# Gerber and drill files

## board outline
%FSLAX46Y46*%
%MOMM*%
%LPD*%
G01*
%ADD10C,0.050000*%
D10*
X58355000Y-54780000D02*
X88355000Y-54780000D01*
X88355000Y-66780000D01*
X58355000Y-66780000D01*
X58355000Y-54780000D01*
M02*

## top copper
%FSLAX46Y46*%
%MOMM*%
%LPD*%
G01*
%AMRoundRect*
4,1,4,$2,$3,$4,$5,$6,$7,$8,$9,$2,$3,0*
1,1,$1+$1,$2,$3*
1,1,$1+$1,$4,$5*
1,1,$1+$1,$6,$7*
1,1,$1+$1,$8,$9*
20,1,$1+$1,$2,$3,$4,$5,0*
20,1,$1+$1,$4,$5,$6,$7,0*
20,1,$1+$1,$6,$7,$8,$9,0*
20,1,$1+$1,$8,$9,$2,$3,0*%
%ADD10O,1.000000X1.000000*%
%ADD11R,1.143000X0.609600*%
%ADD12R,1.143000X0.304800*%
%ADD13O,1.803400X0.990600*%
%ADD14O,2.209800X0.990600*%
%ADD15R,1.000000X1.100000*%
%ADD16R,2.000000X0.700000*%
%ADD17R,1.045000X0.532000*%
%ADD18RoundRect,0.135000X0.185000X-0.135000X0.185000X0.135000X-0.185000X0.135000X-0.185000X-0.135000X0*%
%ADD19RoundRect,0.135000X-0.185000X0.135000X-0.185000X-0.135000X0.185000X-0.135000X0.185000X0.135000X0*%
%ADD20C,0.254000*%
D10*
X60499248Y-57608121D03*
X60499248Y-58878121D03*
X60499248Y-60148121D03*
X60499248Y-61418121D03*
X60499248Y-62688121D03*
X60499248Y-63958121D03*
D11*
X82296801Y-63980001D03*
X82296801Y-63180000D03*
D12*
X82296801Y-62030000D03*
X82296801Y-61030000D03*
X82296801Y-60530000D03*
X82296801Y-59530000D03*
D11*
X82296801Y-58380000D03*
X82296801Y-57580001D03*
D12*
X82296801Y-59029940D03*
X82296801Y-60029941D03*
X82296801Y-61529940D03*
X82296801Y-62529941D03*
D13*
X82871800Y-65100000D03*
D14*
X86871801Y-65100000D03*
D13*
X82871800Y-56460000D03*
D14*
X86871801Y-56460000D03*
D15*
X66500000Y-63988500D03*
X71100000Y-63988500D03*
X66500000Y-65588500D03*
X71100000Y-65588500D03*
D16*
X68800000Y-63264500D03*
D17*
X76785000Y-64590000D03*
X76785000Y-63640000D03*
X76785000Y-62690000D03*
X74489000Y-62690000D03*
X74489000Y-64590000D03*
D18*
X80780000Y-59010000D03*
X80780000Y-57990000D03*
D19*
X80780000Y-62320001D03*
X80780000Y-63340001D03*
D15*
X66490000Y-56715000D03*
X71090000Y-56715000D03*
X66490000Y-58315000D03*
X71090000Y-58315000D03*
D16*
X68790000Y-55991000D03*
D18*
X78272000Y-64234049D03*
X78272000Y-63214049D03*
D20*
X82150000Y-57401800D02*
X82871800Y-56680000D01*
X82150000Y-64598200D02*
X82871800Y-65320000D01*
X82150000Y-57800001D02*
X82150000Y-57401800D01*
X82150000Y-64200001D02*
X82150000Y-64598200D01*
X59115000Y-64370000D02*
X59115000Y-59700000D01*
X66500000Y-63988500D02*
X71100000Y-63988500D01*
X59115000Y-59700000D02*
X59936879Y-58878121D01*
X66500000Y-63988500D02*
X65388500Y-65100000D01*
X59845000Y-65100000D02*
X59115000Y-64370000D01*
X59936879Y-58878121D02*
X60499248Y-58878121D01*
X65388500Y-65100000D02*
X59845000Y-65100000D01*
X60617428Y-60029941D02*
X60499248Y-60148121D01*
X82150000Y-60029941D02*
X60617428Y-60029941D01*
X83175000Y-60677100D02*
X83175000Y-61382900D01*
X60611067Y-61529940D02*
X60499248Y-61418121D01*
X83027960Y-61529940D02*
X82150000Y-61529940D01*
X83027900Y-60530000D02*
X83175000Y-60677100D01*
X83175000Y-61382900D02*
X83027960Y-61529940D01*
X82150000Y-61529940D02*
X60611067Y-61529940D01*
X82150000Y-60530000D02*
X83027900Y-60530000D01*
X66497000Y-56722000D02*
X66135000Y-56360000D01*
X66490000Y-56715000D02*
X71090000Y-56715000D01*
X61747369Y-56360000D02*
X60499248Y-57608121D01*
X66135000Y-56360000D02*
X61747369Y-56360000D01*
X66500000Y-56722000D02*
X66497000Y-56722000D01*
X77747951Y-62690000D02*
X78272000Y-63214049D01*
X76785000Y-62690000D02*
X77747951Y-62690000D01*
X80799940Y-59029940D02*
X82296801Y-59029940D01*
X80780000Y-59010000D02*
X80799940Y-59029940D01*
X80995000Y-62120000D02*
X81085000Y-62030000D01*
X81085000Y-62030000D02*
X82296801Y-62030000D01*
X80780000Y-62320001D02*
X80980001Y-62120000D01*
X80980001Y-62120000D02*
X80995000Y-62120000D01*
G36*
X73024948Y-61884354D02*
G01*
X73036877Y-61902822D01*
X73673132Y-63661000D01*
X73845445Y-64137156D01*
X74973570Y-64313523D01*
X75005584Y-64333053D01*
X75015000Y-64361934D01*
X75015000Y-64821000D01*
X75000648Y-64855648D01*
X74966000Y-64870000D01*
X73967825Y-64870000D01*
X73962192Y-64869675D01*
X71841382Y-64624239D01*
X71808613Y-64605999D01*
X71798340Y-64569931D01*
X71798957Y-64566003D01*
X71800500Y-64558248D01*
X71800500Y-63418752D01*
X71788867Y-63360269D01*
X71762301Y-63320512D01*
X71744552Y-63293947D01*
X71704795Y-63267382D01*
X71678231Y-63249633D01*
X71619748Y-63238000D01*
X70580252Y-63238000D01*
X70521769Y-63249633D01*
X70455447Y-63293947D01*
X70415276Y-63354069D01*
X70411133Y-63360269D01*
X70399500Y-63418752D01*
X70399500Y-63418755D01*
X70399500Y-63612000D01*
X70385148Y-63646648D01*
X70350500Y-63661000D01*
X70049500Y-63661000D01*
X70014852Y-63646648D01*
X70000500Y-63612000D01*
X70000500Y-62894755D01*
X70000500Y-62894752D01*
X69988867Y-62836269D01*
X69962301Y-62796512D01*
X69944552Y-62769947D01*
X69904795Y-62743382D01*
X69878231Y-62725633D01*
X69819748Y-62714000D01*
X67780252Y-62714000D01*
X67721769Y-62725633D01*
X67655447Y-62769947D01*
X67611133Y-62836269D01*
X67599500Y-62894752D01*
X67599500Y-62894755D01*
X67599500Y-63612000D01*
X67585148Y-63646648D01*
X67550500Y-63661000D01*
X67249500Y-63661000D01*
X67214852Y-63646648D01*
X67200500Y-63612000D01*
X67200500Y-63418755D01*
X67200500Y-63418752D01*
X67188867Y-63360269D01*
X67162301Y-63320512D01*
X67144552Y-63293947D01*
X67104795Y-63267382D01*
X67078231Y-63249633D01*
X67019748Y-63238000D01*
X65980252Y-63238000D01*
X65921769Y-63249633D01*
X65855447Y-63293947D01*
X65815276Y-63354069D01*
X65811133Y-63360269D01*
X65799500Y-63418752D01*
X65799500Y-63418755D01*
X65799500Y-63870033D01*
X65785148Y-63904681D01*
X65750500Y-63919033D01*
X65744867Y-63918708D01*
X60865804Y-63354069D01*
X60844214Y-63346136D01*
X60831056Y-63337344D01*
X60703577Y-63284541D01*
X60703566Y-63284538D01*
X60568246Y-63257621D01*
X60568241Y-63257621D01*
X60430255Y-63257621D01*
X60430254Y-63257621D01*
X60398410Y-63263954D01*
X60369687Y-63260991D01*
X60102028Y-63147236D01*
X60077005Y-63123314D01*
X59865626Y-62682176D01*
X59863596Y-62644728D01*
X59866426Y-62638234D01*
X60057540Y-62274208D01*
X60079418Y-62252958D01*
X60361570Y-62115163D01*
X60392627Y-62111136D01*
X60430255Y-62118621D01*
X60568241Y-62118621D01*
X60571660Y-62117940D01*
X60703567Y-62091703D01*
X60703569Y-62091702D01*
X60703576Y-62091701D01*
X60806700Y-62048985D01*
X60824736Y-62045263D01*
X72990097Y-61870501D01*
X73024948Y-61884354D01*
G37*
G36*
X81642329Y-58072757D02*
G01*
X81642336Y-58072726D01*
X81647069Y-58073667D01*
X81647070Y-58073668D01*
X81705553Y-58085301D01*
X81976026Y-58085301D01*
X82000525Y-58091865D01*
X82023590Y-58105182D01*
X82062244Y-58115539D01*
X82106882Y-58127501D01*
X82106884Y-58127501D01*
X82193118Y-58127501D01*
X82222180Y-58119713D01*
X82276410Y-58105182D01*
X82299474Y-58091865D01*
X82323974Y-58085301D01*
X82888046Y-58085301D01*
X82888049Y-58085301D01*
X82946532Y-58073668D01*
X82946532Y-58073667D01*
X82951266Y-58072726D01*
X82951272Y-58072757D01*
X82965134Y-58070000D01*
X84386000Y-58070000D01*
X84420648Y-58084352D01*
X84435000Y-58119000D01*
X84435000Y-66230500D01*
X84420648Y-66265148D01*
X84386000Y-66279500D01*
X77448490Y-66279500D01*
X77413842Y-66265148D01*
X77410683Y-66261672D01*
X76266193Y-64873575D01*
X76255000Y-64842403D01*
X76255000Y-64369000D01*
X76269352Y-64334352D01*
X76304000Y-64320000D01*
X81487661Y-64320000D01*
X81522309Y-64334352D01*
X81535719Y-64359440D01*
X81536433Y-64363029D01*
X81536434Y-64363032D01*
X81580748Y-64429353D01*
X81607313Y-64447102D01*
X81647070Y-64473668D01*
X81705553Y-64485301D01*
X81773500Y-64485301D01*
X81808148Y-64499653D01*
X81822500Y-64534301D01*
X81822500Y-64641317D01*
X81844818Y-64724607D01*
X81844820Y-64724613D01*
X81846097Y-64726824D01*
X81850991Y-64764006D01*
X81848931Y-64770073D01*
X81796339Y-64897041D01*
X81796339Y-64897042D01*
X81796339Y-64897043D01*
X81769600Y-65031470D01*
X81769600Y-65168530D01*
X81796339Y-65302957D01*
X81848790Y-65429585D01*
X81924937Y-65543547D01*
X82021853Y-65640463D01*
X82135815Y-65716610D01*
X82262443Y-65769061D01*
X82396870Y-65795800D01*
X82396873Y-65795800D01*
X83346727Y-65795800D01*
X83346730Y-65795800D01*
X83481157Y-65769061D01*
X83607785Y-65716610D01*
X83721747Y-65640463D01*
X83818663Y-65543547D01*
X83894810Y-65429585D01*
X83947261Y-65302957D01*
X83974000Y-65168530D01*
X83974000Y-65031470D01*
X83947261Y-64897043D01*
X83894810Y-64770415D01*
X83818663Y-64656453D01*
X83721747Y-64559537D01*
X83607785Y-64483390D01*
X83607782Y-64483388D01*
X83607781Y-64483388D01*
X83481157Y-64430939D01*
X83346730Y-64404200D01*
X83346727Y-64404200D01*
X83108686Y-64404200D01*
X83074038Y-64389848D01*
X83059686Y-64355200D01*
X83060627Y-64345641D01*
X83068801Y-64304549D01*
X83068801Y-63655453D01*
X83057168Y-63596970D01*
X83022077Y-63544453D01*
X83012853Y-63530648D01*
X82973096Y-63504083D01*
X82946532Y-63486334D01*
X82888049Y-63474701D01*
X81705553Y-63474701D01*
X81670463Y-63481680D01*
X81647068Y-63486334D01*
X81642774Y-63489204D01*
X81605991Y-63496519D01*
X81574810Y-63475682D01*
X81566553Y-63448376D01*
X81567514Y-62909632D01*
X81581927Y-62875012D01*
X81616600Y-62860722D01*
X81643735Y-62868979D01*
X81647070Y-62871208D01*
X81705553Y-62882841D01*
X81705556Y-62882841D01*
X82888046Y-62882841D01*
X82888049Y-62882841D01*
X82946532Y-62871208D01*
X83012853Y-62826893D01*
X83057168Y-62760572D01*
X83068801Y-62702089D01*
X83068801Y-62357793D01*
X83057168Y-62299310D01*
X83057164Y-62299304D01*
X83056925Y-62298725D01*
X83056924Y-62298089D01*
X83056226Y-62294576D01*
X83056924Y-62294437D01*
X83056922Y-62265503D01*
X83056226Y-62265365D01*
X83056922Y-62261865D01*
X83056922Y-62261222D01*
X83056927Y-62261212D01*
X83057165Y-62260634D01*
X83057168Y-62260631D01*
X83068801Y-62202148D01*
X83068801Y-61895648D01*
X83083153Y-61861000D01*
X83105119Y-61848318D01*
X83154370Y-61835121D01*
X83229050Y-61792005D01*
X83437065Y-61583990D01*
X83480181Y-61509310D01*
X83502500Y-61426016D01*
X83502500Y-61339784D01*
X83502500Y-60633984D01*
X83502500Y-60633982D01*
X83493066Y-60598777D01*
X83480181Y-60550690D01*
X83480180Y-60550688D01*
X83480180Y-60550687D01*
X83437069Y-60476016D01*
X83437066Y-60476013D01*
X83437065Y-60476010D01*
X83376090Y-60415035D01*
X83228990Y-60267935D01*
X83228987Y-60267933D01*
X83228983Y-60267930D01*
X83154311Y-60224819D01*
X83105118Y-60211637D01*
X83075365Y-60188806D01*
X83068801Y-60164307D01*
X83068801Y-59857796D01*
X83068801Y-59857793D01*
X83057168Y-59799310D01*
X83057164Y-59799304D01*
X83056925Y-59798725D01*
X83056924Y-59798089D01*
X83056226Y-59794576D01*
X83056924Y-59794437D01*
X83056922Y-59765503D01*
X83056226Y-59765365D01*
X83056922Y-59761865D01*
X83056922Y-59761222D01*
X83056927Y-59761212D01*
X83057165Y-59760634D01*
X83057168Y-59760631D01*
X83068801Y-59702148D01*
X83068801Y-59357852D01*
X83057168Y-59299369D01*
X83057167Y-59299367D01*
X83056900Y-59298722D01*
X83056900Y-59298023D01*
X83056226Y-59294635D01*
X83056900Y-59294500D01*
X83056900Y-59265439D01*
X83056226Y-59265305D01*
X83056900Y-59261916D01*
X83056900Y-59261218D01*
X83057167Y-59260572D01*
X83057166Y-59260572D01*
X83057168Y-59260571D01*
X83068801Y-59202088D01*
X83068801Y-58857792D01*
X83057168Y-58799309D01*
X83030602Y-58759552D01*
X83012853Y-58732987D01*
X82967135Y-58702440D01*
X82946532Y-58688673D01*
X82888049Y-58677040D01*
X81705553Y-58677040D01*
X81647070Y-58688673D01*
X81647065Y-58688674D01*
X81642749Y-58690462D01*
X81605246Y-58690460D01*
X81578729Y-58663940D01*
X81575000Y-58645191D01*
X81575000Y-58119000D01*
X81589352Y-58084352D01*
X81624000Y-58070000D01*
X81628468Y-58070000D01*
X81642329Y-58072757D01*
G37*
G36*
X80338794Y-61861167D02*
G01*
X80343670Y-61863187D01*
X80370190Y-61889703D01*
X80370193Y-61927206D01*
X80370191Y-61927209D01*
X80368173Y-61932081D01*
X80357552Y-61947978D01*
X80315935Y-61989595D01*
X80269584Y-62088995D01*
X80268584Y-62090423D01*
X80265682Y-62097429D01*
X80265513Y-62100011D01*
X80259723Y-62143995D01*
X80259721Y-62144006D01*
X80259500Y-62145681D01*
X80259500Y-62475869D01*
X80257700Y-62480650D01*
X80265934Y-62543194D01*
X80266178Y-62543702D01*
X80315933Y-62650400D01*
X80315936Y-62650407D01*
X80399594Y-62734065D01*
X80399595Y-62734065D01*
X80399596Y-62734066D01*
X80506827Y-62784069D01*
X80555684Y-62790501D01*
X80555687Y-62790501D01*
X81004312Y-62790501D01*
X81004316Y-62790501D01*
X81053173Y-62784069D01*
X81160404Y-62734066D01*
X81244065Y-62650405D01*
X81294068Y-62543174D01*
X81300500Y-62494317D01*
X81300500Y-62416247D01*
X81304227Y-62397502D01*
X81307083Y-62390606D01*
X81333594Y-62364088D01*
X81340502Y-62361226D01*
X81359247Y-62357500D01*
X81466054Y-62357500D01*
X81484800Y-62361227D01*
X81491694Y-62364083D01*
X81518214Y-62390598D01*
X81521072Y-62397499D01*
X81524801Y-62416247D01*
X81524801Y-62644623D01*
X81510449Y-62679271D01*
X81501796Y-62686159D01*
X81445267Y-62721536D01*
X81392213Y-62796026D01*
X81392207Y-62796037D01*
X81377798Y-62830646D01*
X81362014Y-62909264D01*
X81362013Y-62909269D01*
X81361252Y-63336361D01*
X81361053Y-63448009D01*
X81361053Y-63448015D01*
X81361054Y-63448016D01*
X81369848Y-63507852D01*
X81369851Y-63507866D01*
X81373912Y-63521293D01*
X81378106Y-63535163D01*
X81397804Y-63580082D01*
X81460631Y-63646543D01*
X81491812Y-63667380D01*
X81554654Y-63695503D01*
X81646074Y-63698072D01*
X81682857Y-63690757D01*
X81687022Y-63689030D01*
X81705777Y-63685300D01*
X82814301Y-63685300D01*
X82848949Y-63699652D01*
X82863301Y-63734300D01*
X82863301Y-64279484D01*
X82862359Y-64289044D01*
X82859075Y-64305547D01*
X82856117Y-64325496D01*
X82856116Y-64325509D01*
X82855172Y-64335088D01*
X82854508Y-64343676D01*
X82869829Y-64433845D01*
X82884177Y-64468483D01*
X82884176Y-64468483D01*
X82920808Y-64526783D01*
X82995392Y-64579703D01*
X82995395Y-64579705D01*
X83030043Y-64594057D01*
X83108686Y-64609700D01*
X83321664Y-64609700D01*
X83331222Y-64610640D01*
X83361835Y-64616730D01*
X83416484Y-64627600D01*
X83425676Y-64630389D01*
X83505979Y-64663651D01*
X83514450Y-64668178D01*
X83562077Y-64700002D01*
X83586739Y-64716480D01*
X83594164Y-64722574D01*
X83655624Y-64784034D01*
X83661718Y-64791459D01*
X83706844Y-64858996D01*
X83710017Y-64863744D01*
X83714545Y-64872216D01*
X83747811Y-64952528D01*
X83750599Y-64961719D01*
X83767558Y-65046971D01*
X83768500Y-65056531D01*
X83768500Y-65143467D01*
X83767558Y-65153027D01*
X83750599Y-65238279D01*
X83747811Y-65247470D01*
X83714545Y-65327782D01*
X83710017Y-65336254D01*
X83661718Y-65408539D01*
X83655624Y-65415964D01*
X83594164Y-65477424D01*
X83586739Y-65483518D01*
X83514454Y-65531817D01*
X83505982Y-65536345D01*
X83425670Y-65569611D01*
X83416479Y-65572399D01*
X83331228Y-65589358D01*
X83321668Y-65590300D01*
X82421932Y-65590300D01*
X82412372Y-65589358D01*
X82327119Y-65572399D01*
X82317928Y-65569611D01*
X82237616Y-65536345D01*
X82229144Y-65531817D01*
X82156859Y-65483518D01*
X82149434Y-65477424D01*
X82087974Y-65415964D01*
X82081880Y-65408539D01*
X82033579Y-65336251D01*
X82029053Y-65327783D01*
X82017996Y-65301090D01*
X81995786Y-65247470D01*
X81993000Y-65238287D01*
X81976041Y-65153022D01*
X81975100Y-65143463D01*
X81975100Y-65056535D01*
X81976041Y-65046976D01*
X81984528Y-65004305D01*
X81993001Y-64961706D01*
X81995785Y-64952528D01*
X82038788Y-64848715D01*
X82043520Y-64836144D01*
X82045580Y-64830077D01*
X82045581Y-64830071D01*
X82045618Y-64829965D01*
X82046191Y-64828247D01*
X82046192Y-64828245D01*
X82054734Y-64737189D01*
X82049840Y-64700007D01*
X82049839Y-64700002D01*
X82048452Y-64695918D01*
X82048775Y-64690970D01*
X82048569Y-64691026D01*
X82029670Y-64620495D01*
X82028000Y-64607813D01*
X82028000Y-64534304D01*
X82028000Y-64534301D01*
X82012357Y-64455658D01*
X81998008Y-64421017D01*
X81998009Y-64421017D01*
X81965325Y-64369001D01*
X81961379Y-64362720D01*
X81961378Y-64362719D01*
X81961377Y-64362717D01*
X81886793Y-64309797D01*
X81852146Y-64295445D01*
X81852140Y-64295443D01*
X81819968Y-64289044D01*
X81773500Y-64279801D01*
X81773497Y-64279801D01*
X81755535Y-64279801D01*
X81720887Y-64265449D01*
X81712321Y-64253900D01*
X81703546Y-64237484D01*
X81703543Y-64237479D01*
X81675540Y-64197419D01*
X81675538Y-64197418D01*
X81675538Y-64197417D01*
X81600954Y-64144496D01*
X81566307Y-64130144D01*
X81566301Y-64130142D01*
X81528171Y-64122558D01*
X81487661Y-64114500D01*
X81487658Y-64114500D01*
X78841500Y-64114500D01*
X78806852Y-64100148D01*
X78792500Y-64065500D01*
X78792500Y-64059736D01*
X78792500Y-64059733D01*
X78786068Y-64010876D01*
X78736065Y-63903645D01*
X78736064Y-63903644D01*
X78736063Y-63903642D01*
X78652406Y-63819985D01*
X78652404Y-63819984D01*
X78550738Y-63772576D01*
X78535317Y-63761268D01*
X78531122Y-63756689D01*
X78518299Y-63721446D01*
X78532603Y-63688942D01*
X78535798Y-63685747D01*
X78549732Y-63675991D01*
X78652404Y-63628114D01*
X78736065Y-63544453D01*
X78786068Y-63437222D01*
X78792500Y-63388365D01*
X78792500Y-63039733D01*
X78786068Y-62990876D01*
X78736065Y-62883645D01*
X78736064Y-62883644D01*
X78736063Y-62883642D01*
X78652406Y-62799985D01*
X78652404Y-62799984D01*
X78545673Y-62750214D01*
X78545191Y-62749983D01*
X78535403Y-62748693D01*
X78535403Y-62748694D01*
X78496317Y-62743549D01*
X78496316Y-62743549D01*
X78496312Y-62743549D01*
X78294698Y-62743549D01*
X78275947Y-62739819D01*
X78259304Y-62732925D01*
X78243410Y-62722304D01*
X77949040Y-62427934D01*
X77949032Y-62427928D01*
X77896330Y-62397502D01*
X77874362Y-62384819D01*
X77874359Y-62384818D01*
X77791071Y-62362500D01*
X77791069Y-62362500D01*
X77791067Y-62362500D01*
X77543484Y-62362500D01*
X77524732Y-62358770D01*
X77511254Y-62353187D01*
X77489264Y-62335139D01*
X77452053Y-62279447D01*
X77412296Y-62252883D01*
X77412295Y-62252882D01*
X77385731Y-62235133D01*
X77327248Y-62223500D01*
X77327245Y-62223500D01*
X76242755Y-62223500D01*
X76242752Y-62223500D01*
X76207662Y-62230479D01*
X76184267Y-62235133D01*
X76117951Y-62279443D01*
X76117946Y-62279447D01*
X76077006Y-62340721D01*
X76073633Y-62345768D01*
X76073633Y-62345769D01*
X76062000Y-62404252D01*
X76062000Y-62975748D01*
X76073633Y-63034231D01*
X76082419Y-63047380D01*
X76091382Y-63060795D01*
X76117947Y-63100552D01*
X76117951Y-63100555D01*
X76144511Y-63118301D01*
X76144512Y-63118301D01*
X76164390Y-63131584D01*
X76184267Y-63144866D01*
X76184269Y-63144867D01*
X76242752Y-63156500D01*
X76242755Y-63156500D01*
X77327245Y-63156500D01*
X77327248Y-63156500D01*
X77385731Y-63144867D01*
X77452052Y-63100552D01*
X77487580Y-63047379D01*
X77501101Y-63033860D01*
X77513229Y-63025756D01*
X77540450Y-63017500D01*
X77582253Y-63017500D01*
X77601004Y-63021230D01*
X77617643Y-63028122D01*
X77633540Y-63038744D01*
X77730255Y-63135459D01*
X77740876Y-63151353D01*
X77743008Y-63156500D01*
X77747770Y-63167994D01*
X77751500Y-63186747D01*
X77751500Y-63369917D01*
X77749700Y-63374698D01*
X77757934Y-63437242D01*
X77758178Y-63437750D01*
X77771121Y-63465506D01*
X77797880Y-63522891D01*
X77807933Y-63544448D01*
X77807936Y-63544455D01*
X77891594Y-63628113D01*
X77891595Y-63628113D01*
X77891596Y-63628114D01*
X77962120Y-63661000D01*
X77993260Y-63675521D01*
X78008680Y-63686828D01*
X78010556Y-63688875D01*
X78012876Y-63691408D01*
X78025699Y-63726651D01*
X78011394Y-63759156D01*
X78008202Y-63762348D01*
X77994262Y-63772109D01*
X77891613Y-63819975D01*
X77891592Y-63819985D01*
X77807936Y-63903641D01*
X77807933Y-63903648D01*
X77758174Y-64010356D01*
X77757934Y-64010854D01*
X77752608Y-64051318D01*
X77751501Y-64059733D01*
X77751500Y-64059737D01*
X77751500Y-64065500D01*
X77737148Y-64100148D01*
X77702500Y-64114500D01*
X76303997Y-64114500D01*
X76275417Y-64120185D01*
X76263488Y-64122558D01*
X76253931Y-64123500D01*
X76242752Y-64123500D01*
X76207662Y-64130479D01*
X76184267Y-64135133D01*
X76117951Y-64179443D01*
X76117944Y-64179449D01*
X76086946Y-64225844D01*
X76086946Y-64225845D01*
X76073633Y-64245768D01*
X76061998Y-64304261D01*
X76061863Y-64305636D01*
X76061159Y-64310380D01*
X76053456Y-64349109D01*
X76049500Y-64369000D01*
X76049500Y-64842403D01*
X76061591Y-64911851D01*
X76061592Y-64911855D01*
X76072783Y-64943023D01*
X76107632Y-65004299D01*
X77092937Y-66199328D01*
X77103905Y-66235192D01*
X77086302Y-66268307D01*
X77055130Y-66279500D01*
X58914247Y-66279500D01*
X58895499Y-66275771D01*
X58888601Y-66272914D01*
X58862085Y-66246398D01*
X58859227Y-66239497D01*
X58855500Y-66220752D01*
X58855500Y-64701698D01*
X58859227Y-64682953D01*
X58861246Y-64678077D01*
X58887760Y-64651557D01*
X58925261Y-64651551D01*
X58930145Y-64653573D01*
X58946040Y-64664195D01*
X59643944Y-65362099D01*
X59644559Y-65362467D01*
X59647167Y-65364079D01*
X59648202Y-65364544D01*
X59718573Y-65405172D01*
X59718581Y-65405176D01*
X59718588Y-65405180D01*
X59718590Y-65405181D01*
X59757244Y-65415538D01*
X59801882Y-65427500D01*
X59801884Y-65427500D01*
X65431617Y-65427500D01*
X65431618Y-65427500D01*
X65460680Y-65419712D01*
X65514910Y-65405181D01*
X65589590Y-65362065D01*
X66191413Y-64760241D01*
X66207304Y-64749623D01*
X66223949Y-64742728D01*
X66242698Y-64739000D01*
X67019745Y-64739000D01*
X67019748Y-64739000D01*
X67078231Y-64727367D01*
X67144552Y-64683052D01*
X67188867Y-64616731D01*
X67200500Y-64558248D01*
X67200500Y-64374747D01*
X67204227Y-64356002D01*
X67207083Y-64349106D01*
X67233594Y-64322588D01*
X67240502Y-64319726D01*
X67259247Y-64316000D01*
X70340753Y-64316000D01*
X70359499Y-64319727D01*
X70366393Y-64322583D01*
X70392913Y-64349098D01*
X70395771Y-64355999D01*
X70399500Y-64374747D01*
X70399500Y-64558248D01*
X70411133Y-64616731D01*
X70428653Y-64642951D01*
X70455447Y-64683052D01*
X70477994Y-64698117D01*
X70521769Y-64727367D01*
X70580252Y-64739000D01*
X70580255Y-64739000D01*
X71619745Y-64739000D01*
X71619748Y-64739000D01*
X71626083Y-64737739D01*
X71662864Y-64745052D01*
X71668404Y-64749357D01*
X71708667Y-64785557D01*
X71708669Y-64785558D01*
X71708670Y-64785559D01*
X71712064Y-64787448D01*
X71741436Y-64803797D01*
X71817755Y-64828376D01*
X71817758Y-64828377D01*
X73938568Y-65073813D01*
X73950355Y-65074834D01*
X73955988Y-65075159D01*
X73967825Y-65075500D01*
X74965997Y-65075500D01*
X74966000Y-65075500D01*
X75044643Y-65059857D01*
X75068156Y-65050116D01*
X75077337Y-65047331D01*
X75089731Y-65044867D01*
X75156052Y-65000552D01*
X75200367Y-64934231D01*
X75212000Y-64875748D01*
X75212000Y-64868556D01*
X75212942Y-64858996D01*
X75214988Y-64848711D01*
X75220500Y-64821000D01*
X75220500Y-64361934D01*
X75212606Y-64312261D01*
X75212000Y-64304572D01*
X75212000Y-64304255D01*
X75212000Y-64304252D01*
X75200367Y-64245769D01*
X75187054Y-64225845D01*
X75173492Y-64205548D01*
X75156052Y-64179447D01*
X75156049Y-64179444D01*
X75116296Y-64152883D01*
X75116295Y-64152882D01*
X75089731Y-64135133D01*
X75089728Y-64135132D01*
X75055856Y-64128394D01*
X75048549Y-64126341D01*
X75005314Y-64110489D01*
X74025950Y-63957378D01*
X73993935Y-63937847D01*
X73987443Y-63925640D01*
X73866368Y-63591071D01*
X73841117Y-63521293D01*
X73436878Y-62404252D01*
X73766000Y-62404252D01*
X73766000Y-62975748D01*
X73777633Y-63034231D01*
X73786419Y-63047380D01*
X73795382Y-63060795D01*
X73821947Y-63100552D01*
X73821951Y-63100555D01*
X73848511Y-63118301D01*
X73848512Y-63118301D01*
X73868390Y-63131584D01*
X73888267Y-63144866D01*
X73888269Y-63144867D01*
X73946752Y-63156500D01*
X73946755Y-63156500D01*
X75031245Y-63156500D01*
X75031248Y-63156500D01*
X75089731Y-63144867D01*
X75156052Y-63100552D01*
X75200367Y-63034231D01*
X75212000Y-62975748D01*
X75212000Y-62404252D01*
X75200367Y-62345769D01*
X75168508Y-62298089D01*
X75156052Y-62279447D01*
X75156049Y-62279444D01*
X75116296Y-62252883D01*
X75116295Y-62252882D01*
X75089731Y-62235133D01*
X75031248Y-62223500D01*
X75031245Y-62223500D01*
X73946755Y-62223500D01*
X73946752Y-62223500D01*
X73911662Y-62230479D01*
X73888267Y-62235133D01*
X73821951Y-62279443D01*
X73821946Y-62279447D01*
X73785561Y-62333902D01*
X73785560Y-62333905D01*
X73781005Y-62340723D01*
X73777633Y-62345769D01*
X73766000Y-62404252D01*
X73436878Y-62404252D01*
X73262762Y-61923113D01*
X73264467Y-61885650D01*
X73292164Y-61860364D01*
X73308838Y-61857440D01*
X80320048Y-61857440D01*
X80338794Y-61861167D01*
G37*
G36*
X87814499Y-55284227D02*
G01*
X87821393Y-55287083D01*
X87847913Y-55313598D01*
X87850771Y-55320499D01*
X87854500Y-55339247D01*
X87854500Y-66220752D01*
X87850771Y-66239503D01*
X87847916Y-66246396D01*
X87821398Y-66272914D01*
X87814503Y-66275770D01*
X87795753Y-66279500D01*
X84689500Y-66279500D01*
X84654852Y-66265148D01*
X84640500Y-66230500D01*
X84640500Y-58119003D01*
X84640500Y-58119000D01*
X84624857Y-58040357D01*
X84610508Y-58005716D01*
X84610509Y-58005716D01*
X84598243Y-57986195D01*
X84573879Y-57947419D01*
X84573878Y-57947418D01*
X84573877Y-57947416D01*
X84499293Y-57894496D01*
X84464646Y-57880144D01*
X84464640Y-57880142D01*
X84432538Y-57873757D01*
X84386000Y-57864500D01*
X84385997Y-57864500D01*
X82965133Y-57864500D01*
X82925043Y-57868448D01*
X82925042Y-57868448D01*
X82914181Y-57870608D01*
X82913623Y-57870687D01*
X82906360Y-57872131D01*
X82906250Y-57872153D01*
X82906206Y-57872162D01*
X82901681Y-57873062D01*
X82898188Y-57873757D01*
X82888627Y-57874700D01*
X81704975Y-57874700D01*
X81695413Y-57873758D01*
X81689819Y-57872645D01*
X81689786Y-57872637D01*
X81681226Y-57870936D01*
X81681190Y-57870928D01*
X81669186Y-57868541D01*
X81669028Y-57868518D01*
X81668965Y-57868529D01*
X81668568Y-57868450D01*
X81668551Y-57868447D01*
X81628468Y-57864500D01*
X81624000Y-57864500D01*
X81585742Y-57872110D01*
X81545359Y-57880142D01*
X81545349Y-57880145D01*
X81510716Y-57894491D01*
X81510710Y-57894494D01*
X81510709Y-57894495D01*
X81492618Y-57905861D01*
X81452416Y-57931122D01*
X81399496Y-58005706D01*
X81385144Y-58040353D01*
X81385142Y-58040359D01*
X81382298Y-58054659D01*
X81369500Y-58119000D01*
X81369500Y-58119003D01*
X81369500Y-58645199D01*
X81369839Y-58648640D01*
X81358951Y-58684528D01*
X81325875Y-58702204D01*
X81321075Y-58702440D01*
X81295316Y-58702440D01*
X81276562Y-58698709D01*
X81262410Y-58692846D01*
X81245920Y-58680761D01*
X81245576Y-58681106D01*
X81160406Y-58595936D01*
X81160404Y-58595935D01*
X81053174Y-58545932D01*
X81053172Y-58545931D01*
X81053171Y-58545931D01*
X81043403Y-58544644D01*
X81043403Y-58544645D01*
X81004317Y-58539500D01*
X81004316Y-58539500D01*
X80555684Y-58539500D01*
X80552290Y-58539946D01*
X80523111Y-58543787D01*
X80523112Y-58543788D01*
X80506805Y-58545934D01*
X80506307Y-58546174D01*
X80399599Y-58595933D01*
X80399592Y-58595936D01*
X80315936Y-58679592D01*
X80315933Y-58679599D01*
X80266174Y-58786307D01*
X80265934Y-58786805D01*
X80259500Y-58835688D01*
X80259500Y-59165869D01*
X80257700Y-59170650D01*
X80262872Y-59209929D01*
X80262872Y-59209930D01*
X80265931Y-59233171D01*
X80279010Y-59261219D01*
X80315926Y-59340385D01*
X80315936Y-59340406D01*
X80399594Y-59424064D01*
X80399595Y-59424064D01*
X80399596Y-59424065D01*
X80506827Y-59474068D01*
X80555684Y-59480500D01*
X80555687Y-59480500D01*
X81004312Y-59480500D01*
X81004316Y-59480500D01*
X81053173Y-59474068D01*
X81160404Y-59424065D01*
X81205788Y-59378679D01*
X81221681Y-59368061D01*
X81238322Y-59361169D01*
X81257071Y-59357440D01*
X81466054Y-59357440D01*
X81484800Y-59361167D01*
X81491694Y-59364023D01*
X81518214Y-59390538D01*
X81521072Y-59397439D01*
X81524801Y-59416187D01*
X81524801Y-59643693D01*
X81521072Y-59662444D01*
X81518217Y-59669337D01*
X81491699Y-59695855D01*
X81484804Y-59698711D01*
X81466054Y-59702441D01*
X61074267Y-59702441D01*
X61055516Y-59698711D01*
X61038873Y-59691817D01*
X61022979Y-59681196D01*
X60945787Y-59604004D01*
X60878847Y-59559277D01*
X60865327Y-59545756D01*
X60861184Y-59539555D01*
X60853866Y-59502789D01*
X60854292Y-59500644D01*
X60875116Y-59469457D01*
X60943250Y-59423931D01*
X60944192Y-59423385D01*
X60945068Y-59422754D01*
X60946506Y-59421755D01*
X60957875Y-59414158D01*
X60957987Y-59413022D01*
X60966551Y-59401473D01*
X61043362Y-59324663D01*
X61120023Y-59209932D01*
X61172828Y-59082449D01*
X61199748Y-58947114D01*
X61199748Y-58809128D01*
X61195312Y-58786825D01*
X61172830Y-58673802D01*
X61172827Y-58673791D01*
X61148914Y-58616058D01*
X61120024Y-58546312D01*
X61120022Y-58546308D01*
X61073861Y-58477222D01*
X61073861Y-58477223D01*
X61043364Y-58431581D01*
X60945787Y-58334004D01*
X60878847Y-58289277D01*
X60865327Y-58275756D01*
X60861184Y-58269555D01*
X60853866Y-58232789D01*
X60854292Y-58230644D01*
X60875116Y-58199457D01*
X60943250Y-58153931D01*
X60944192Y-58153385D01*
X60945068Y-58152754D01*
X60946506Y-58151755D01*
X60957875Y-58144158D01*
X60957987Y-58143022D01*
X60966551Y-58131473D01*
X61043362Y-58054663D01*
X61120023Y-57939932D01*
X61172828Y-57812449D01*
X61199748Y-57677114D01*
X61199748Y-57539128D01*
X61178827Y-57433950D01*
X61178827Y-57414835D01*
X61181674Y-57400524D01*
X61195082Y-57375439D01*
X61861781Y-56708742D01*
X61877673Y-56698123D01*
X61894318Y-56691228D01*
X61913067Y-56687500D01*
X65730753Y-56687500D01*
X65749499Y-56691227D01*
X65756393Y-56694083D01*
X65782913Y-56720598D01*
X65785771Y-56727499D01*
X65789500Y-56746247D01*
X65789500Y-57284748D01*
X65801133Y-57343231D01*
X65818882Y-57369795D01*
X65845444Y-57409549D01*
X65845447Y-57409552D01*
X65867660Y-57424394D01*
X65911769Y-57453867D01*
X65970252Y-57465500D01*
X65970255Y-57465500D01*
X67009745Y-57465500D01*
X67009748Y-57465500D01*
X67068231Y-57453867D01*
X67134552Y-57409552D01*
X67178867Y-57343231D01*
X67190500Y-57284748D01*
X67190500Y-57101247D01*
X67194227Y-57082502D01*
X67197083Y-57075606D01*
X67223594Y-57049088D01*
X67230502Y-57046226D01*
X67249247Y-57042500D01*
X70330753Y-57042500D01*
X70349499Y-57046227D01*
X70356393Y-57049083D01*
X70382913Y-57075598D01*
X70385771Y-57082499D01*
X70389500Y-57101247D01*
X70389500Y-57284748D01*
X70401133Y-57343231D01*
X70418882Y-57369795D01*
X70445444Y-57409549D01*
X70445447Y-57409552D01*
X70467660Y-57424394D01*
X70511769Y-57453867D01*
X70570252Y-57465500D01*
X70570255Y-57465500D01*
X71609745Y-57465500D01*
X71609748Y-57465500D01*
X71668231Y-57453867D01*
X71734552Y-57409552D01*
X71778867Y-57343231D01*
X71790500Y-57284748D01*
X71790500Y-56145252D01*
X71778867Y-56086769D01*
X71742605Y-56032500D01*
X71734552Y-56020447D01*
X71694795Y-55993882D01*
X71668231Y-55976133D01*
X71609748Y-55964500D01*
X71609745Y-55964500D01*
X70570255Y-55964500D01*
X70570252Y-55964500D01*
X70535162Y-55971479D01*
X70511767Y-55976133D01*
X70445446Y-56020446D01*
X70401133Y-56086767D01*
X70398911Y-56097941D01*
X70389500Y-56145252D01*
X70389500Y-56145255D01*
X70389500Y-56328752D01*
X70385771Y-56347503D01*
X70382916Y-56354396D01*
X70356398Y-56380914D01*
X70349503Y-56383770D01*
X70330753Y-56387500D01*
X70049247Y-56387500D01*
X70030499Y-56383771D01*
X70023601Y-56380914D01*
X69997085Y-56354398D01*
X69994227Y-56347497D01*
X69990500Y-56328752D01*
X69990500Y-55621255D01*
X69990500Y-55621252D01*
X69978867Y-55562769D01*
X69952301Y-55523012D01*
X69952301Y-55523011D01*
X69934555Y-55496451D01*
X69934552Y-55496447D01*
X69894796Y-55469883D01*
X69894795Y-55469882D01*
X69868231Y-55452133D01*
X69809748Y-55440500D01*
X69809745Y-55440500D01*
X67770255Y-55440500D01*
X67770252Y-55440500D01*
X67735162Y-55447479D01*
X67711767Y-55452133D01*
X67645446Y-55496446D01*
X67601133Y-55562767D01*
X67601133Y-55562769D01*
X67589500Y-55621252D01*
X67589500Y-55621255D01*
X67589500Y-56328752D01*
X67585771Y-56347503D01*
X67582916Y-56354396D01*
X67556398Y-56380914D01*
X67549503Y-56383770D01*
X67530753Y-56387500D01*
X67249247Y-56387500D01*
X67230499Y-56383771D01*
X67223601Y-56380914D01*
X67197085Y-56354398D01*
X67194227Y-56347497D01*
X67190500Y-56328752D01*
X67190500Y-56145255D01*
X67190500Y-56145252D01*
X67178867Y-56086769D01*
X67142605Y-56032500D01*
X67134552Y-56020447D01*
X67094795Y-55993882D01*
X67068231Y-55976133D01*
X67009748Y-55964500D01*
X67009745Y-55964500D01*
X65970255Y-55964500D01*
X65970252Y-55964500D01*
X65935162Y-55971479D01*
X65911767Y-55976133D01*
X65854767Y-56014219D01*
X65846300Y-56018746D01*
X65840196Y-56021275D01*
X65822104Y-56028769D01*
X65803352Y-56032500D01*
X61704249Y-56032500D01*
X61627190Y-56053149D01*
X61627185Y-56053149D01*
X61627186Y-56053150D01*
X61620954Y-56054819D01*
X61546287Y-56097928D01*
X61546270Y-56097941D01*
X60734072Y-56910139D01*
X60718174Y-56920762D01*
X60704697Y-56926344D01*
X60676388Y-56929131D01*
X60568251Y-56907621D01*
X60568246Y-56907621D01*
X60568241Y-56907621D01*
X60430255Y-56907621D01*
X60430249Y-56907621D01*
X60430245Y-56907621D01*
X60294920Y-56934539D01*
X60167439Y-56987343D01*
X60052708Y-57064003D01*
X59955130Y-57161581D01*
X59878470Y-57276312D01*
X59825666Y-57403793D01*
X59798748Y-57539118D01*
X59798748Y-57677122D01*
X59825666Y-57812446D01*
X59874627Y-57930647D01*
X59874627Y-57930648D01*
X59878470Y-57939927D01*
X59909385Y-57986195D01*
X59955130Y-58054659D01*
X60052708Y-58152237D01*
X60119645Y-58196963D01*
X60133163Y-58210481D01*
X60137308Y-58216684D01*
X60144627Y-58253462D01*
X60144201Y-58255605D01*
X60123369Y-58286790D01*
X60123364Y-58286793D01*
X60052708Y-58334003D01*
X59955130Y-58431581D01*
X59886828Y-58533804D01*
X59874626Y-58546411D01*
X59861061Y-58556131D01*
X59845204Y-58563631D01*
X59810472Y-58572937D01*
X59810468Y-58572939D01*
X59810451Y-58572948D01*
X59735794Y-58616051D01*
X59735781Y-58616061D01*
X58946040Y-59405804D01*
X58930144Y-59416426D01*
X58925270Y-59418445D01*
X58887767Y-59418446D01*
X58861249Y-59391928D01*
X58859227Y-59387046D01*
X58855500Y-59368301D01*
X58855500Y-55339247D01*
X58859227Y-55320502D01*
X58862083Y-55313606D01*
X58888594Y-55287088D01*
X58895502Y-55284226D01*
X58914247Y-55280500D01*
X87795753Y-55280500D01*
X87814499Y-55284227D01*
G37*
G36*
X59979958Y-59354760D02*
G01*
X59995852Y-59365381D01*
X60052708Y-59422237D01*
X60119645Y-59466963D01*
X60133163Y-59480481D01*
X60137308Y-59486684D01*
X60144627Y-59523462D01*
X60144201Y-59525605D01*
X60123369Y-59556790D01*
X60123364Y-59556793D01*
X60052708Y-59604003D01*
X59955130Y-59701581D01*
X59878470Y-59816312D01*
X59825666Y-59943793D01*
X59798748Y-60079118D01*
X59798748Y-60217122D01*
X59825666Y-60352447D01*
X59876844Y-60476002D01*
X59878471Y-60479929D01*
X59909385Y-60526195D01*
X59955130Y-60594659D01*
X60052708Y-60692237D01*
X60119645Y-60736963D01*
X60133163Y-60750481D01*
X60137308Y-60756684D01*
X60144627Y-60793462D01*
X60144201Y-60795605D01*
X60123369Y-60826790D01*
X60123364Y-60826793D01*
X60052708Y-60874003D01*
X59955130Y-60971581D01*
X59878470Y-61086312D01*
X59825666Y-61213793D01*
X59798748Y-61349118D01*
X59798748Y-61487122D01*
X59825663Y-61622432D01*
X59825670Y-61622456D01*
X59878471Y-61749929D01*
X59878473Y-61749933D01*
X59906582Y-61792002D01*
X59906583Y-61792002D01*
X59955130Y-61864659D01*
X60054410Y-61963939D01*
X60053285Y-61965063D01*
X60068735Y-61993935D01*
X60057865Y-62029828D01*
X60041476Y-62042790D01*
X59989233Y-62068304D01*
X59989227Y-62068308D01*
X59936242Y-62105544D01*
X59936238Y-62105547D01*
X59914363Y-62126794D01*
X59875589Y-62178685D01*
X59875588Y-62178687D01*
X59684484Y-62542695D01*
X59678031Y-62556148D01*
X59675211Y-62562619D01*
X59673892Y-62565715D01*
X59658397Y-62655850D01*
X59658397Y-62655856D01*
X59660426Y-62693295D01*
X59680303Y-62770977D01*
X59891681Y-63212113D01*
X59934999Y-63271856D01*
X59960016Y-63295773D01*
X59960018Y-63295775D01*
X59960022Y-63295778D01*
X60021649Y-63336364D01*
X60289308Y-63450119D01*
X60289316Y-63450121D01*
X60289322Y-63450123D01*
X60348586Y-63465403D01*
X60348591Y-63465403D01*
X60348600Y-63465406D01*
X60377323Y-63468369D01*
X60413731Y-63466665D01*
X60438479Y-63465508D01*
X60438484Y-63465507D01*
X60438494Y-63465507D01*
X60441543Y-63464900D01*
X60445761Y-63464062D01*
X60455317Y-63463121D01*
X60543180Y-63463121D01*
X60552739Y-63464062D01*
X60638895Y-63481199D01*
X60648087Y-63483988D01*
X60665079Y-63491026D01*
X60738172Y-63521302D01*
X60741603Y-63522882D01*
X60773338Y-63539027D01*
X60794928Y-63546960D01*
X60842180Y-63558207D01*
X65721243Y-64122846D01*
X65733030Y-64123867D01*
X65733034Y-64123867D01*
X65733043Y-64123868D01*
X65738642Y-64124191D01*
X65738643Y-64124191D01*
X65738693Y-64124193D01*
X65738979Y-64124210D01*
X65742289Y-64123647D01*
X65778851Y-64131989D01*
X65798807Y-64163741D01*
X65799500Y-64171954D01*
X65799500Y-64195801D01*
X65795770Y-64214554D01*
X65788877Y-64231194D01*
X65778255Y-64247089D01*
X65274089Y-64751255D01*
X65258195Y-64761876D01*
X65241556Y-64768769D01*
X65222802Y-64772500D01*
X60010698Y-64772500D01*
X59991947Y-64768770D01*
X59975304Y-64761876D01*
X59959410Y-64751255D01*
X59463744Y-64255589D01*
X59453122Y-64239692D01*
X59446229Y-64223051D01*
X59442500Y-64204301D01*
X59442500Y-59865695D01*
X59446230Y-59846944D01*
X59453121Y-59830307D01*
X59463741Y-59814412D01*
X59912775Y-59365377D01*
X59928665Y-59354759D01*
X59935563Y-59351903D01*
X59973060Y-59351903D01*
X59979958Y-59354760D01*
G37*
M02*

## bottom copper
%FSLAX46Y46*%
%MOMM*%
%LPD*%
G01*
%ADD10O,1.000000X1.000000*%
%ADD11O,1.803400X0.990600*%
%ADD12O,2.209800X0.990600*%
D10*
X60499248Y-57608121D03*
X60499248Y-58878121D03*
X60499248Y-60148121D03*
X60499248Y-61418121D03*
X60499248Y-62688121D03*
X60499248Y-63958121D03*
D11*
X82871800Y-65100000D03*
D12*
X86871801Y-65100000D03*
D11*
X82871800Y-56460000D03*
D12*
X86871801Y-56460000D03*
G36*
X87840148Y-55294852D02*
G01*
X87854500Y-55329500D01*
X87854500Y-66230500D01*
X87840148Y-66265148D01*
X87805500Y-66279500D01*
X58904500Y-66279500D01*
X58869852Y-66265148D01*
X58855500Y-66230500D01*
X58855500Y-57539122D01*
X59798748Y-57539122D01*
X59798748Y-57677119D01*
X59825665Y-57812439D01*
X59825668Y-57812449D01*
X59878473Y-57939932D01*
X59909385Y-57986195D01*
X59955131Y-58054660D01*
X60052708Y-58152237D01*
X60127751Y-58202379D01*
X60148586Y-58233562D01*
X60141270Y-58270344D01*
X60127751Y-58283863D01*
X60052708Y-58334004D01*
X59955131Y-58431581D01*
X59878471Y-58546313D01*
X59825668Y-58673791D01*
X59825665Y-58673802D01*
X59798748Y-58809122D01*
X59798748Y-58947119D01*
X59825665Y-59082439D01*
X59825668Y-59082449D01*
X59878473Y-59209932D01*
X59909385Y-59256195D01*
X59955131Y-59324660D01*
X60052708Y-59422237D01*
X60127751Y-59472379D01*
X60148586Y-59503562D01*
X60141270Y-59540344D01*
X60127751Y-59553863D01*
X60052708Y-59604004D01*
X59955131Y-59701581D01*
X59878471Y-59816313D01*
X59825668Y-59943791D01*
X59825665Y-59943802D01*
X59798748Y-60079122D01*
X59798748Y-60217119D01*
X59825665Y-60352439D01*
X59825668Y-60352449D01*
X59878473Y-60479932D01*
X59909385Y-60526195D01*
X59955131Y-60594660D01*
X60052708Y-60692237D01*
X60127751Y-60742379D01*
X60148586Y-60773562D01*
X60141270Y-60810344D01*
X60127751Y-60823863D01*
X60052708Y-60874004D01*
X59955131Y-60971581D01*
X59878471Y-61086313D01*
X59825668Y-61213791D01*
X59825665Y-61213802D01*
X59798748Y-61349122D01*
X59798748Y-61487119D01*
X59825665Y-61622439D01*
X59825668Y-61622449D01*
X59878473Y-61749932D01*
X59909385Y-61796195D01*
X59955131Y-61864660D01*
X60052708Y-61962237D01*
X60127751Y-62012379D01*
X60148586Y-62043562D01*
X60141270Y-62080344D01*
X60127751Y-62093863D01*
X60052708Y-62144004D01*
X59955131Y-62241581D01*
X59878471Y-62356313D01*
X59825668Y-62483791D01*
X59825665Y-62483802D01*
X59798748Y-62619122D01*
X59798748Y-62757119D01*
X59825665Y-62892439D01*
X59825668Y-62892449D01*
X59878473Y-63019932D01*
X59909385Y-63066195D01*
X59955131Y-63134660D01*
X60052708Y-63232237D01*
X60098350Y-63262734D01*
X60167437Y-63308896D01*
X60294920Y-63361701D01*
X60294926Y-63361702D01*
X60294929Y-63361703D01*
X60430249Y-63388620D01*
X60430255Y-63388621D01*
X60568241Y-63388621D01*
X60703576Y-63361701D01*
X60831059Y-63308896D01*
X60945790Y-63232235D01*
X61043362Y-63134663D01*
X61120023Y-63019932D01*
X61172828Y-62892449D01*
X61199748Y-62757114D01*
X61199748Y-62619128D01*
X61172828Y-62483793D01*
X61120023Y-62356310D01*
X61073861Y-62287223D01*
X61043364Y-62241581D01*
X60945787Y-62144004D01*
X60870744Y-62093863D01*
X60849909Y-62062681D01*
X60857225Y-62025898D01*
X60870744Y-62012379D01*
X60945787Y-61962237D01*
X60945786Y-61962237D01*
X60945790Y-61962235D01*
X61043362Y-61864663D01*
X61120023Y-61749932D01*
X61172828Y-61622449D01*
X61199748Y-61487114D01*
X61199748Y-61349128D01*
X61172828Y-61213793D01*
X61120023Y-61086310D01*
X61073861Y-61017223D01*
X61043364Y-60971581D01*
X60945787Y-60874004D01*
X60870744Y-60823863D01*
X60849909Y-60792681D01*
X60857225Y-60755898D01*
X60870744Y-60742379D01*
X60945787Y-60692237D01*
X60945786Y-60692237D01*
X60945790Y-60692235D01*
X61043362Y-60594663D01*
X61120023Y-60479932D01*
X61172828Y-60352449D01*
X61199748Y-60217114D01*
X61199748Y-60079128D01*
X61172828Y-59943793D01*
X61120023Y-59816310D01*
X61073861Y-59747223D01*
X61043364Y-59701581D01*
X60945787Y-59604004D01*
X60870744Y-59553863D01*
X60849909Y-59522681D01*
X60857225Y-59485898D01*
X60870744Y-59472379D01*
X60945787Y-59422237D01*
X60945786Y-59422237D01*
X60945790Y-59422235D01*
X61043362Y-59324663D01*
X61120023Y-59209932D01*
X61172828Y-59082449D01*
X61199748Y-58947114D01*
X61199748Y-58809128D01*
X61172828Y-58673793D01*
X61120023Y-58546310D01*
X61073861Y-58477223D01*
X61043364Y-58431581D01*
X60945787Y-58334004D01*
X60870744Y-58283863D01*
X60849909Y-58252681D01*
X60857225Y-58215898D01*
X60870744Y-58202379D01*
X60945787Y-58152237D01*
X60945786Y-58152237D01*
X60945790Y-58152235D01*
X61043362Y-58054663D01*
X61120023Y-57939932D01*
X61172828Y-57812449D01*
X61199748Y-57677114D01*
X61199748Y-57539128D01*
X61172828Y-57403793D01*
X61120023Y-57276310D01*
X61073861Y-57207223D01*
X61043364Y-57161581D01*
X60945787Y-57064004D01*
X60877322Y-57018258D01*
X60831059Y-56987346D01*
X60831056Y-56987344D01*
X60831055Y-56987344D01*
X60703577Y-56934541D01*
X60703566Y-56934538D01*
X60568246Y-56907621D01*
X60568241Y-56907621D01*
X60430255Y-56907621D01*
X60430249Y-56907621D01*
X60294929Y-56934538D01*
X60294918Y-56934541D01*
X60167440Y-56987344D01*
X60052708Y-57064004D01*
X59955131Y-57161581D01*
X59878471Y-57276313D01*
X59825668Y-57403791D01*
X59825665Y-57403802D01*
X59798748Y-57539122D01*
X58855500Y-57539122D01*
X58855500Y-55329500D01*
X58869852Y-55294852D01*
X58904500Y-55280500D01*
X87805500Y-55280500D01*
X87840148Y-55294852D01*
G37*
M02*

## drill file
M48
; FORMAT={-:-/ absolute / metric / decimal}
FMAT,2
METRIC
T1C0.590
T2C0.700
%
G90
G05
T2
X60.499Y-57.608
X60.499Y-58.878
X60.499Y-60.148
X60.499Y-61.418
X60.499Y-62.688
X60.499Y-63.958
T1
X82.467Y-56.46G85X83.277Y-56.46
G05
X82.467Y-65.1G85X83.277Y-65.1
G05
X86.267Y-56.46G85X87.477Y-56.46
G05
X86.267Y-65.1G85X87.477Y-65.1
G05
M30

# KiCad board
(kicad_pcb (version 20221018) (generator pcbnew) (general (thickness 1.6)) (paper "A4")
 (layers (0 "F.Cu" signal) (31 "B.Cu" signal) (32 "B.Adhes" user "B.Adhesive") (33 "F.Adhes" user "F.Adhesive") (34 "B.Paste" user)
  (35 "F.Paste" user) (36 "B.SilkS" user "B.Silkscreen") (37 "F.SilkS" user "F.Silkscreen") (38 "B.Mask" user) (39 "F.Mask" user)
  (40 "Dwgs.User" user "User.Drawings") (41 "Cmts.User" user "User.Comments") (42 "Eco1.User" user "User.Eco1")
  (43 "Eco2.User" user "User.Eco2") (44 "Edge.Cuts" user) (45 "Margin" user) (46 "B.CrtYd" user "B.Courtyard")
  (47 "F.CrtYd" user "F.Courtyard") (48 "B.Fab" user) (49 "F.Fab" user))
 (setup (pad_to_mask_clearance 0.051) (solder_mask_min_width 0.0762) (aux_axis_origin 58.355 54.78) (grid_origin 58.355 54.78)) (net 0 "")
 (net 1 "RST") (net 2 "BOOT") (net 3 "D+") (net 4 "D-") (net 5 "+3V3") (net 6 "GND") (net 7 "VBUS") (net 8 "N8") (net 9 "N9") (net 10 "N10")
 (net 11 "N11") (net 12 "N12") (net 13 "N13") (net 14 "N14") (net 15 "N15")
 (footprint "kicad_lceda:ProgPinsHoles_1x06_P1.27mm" (layer "F.Cu") (at 60.499248 57.608121)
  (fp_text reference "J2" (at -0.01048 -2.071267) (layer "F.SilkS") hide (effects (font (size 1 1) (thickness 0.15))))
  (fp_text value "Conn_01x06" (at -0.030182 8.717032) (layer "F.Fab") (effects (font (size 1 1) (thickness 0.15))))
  (pad "1" thru_hole oval (at 0 0) (size 1 1) (drill 0.7) (layers "*.Cu" "*.Mask") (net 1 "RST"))
  (pad "2" thru_hole oval (at 0 1.27) (size 1 1) (drill 0.7) (layers "*.Cu" "*.Mask") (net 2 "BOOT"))
  (pad "3" thru_hole oval (at 0 2.54) (size 1 1) (drill 0.7) (layers "*.Cu" "*.Mask") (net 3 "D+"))
  (pad "4" thru_hole oval (at 0 3.81) (size 1 1) (drill 0.7) (layers "*.Cu" "*.Mask") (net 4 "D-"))
  (pad "5" thru_hole oval (at 0 5.08) (size 1 1) (drill 0.7) (layers "*.Cu" "*.Mask") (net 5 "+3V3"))
  (pad "6" thru_hole oval (at 0 6.35) (size 1 1) (drill 0.7) (layers "*.Cu" "*.Mask") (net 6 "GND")))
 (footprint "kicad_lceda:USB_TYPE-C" (layer "F.Cu") (at 85.6 60.78 90)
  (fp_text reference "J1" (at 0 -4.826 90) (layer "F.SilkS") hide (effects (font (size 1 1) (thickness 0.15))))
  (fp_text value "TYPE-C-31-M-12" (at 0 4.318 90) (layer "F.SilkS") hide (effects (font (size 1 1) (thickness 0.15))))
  (pad "A1" smd rect (at -3.200001 -3.303199 90) (size 0.6096 1.143) (layers "F.Cu" "F.Paste" "F.Mask") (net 6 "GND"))
  (pad "A4" smd rect (at -2.4 -3.303199 90) (size 0.6096 1.143) (layers "F.Cu" "F.Paste" "F.Mask") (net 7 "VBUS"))
  (pad "A5" smd rect (at -1.25 -3.303199 90) (size 0.3048 1.143) (layers "F.Cu" "F.Paste" "F.Mask") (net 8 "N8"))
  (pad "A6" smd rect (at -0.25 -3.303199 90) (size 0.3048 1.143) (layers "F.Cu" "F.Paste" "F.Mask") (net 3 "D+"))
  (pad "A7" smd rect (at 0.25 -3.303199 90) (size 0.3048 1.143) (layers "F.Cu" "F.Paste" "F.Mask") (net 4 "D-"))
  (pad "A8" smd rect (at 1.25 -3.303199 90) (size 0.3048 1.143) (layers "F.Cu" "F.Paste" "F.Mask") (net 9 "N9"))
  (pad "A9" smd rect (at 2.4 -3.303199 90) (size 0.6096 1.143) (layers "F.Cu" "F.Paste" "F.Mask") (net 7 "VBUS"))
  (pad "A12" smd rect (at 3.199999 -3.303199 90) (size 0.6096 1.143) (layers "F.Cu" "F.Paste" "F.Mask") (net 6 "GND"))
  (pad "B5" smd rect (at 1.75006 -3.303199 90) (size 0.3048 1.143) (layers "F.Cu" "F.Paste" "F.Mask") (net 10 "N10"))
  (pad "B6" smd rect (at 0.750059 -3.303199 90) (size 0.3048 1.143) (layers "F.Cu" "F.Paste" "F.Mask") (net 3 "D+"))
  (pad "B7" smd rect (at -0.74994 -3.303199 90) (size 0.3048 1.143) (layers "F.Cu" "F.Paste" "F.Mask") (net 4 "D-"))
  (pad "B8" smd rect (at -1.749941 -3.303199 90) (size 0.3048 1.143) (layers "F.Cu" "F.Paste" "F.Mask") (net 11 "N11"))
  (pad "S1" thru_hole oval (at -4.32 -2.7282 90) (size 0.9906 1.8034) (drill oval 0.59 1.4) (layers "*.Cu" "*.Mask") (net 6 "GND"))
  (pad "S1" thru_hole oval (at -4.32 1.271801 90) (size 0.9906 2.2098) (drill oval 0.59 1.8) (layers "*.Cu" "*.Mask") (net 6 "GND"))
  (pad "S1" thru_hole oval (at 4.32 -2.7282 90) (size 0.9906 1.8034) (drill oval 0.59 1.4) (layers "*.Cu" "*.Mask") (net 6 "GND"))
  (pad "S1" thru_hole oval (at 4.32 1.271801 90) (size 0.9906 2.2098) (drill oval 0.59 1.8) (layers "*.Cu" "*.Mask") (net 6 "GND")))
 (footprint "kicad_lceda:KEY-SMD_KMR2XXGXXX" (layer "F.Cu") (at 68.8 64.4265)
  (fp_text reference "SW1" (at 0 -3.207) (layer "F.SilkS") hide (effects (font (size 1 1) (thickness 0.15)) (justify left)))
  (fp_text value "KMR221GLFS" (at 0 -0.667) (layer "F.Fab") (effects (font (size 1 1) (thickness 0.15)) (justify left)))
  (pad "1" smd rect (at -2.3 -0.438) (size 1 1.1) (layers "F.Cu" "F.Paste" "F.Mask") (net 2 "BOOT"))
  (pad "2" smd rect (at 2.3 -0.438) (size 1 1.1) (layers "F.Cu" "F.Paste" "F.Mask") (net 2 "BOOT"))
  (pad "3" smd rect (at -2.3 1.162) (size 1 1.1) (layers "F.Cu" "F.Paste" "F.Mask") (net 6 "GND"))
  (pad "4" smd rect (at 2.3 1.162) (size 1 1.1) (layers "F.Cu" "F.Paste" "F.Mask") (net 6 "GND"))
  (pad "5" smd rect (at 0 -1.162) (size 2 0.7) (layers "F.Cu" "F.Paste" "F.Mask") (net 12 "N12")))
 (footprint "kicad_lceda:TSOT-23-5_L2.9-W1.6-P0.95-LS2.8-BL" (layer "F.Cu") (at 75.637 63.64 90)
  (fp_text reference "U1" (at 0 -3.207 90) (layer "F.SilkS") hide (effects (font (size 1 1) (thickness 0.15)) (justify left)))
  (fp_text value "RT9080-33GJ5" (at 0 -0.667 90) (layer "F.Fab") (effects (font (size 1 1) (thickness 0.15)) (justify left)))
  (pad "1" smd rect (at -0.95 1.148 90) (size 0.532 1.045) (layers "F.Cu" "F.Paste" "F.Mask") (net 7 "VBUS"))
  (pad "2" smd rect (at 0 1.148 90) (size 0.532 1.045) (layers "F.Cu" "F.Paste" "F.Mask") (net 6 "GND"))
  (pad "3" smd rect (at 0.95 1.148 90) (size 0.532 1.045) (layers "F.Cu" "F.Paste" "F.Mask") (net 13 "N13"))
  (pad "4" smd rect (at 0.95 -1.148 90) (size 0.532 1.045) (layers "F.Cu" "F.Paste" "F.Mask") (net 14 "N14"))
  (pad "5" smd rect (at -0.95 -1.148 90) (size 0.532 1.045) (layers "F.Cu" "F.Paste" "F.Mask") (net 5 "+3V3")))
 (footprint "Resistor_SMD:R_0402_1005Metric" (layer "F.Cu") (at 80.78 58.5 90)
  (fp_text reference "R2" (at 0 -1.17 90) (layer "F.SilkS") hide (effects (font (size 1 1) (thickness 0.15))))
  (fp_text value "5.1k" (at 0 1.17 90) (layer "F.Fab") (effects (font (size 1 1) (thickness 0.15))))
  (pad "1" smd roundrect (at -0.51 0 90) (size 0.54 0.64) (layers "F.Cu" "F.Paste" "F.Mask") (roundrect_rratio 0.25) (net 10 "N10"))
  (pad "2" smd roundrect (at 0.51 0 90) (size 0.54 0.64) (layers "F.Cu" "F.Paste" "F.Mask") (roundrect_rratio 0.25) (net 6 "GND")))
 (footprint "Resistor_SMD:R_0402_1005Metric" (layer "F.Cu") (at 80.78 62.830001 -90)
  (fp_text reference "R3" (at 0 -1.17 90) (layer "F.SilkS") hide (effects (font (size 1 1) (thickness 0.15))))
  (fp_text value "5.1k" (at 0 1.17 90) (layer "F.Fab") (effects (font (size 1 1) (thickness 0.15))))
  (pad "1" smd roundrect (at -0.51 0 270) (size 0.54 0.64) (layers "F.Cu" "F.Paste" "F.Mask") (roundrect_rratio 0.25) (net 8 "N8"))
  (pad "2" smd roundrect (at 0.51 0 270) (size 0.54 0.64) (layers "F.Cu" "F.Paste" "F.Mask") (roundrect_rratio 0.25) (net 6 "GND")))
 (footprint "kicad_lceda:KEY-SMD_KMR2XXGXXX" (layer "F.Cu") (at 68.79 57.153)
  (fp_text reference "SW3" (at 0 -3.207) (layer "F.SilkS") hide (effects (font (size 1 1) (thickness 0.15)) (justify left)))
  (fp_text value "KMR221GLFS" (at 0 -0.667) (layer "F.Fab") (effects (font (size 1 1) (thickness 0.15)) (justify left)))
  (pad "1" smd rect (at -2.3 -0.438) (size 1 1.1) (layers "F.Cu" "F.Paste" "F.Mask") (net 1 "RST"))
  (pad "2" smd rect (at 2.3 -0.438) (size 1 1.1) (layers "F.Cu" "F.Paste" "F.Mask") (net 1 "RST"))
  (pad "3" smd rect (at -2.3 1.162) (size 1 1.1) (layers "F.Cu" "F.Paste" "F.Mask") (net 6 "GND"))
  (pad "4" smd rect (at 2.3 1.162) (size 1 1.1) (layers "F.Cu" "F.Paste" "F.Mask") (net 6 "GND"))
  (pad "5" smd rect (at 0 -1.162) (size 2 0.7) (layers "F.Cu" "F.Paste" "F.Mask") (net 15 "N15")))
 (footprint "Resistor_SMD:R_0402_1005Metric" (layer "F.Cu") (at 78.272 63.724049 90)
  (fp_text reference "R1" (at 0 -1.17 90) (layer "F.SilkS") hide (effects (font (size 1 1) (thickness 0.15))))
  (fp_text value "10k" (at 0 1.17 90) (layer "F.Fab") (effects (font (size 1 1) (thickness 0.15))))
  (pad "1" smd roundrect (at -0.51 0 90) (size 0.54 0.64) (layers "F.Cu" "F.Paste" "F.Mask") (roundrect_rratio 0.25) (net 7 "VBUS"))
  (pad "2" smd roundrect (at 0.51 0 90) (size 0.54 0.64) (layers "F.Cu" "F.Paste" "F.Mask") (roundrect_rratio 0.25) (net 13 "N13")))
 (gr_rect (start 58.355 54.78) (end 88.355 66.78) (stroke (width 0.05) (type default)) (fill none) (layer "Edge.Cuts"))
 (segment (start 82.15 57.4018) (end 82.8718 56.68) (width 0.254) (layer "F.Cu") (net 6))
 (segment (start 82.15 64.5982) (end 82.8718 65.32) (width 0.254) (layer "F.Cu") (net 6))
 (segment (start 82.15 57.800001) (end 82.15 57.4018) (width 0.254) (layer "F.Cu") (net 6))
 (segment (start 82.15 64.200001) (end 82.15 64.5982) (width 0.254) (layer "F.Cu") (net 6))
 (segment (start 59.115 64.37) (end 59.115 59.7) (width 0.254) (layer "F.Cu") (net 2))
 (segment (start 66.5 63.9885) (end 71.1 63.9885) (width 0.254) (layer "F.Cu") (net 2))
 (segment (start 59.115 59.7) (end 59.936879 58.878121) (width 0.254) (layer "F.Cu") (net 2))
 (segment (start 66.5 63.9885) (end 65.3885 65.1) (width 0.254) (layer "F.Cu") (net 2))
 (segment (start 59.845 65.1) (end 59.115 64.37) (width 0.254) (layer "F.Cu") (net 2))
 (segment (start 59.936879 58.878121) (end 60.499248 58.878121) (width 0.254) (layer "F.Cu") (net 2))
 (segment (start 65.3885 65.1) (end 59.845 65.1) (width 0.254) (layer "F.Cu") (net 2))
 (segment (start 60.617428 60.029941) (end 60.499248 60.148121) (width 0.254) (layer "F.Cu") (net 3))
 (segment (start 82.15 60.029941) (end 60.617428 60.029941) (width 0.254) (layer "F.Cu") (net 3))
 (segment (start 83.175 60.6771) (end 83.175 61.3829) (width 0.254) (layer "F.Cu") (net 4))
 (segment (start 60.611067 61.52994) (end 60.499248 61.418121) (width 0.254) (layer "F.Cu") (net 4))
 (segment (start 83.02796 61.52994) (end 82.15 61.52994) (width 0.254) (layer "F.Cu") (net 4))
 (segment (start 83.0279 60.53) (end 83.175 60.6771) (width 0.254) (layer "F.Cu") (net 4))
 (segment (start 83.175 61.3829) (end 83.02796 61.52994) (width 0.254) (layer "F.Cu") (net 4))
 (segment (start 82.15 61.52994) (end 60.611067 61.52994) (width 0.254) (layer "F.Cu") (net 4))
 (segment (start 82.15 60.53) (end 83.0279 60.53) (width 0.254) (layer "F.Cu") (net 4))
 (segment (start 66.497 56.722) (end 66.135 56.36) (width 0.254) (layer "F.Cu") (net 1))
 (segment (start 66.49 56.715) (end 71.09 56.715) (width 0.254) (layer "F.Cu") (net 1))
 (segment (start 61.747369 56.36) (end 60.499248 57.608121) (width 0.254) (layer "F.Cu") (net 1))
 (segment (start 66.135 56.36) (end 61.747369 56.36) (width 0.254) (layer "F.Cu") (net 1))
 (segment (start 66.5 56.722) (end 66.497 56.722) (width 0.254) (layer "F.Cu") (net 1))
 (segment (start 77.747951 62.69) (end 78.272 63.214049) (width 0.254) (layer "F.Cu") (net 13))
 (segment (start 76.785 62.69) (end 77.747951 62.69) (width 0.254) (layer "F.Cu") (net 13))
 (segment (start 80.79994 59.02994) (end 82.296801 59.02994) (width 0.254) (layer "F.Cu") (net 10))
 (segment (start 80.78 59.01) (end 80.79994 59.02994) (width 0.254) (layer "F.Cu") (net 10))
 (segment (start 80.995 62.12) (end 81.085 62.03) (width 0.254) (layer "F.Cu") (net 8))
 (segment (start 81.085 62.03) (end 82.296801 62.03) (width 0.254) (layer "F.Cu") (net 8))
 (segment (start 80.78 62.320001) (end 80.980001 62.12) (width 0.254) (layer "F.Cu") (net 8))
 (segment (start 80.980001 62.12) (end 80.995 62.12) (width 0.254) (layer "F.Cu") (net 8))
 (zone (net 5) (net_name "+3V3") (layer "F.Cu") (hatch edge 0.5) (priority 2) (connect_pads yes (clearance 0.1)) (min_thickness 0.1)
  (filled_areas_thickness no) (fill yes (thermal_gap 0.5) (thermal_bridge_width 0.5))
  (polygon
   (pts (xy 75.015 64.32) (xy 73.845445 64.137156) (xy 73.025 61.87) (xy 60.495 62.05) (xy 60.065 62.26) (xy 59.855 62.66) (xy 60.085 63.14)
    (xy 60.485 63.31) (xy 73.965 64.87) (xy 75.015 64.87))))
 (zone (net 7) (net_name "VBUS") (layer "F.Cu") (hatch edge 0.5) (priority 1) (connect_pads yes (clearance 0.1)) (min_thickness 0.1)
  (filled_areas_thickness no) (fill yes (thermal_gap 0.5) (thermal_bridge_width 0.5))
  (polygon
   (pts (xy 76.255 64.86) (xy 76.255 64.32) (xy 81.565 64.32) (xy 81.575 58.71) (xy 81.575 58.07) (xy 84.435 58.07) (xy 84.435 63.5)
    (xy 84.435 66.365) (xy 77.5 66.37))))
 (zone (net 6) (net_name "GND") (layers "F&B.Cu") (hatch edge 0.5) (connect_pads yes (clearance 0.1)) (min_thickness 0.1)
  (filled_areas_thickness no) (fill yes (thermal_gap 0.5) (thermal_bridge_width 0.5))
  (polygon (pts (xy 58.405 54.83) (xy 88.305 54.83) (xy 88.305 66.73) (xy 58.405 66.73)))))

